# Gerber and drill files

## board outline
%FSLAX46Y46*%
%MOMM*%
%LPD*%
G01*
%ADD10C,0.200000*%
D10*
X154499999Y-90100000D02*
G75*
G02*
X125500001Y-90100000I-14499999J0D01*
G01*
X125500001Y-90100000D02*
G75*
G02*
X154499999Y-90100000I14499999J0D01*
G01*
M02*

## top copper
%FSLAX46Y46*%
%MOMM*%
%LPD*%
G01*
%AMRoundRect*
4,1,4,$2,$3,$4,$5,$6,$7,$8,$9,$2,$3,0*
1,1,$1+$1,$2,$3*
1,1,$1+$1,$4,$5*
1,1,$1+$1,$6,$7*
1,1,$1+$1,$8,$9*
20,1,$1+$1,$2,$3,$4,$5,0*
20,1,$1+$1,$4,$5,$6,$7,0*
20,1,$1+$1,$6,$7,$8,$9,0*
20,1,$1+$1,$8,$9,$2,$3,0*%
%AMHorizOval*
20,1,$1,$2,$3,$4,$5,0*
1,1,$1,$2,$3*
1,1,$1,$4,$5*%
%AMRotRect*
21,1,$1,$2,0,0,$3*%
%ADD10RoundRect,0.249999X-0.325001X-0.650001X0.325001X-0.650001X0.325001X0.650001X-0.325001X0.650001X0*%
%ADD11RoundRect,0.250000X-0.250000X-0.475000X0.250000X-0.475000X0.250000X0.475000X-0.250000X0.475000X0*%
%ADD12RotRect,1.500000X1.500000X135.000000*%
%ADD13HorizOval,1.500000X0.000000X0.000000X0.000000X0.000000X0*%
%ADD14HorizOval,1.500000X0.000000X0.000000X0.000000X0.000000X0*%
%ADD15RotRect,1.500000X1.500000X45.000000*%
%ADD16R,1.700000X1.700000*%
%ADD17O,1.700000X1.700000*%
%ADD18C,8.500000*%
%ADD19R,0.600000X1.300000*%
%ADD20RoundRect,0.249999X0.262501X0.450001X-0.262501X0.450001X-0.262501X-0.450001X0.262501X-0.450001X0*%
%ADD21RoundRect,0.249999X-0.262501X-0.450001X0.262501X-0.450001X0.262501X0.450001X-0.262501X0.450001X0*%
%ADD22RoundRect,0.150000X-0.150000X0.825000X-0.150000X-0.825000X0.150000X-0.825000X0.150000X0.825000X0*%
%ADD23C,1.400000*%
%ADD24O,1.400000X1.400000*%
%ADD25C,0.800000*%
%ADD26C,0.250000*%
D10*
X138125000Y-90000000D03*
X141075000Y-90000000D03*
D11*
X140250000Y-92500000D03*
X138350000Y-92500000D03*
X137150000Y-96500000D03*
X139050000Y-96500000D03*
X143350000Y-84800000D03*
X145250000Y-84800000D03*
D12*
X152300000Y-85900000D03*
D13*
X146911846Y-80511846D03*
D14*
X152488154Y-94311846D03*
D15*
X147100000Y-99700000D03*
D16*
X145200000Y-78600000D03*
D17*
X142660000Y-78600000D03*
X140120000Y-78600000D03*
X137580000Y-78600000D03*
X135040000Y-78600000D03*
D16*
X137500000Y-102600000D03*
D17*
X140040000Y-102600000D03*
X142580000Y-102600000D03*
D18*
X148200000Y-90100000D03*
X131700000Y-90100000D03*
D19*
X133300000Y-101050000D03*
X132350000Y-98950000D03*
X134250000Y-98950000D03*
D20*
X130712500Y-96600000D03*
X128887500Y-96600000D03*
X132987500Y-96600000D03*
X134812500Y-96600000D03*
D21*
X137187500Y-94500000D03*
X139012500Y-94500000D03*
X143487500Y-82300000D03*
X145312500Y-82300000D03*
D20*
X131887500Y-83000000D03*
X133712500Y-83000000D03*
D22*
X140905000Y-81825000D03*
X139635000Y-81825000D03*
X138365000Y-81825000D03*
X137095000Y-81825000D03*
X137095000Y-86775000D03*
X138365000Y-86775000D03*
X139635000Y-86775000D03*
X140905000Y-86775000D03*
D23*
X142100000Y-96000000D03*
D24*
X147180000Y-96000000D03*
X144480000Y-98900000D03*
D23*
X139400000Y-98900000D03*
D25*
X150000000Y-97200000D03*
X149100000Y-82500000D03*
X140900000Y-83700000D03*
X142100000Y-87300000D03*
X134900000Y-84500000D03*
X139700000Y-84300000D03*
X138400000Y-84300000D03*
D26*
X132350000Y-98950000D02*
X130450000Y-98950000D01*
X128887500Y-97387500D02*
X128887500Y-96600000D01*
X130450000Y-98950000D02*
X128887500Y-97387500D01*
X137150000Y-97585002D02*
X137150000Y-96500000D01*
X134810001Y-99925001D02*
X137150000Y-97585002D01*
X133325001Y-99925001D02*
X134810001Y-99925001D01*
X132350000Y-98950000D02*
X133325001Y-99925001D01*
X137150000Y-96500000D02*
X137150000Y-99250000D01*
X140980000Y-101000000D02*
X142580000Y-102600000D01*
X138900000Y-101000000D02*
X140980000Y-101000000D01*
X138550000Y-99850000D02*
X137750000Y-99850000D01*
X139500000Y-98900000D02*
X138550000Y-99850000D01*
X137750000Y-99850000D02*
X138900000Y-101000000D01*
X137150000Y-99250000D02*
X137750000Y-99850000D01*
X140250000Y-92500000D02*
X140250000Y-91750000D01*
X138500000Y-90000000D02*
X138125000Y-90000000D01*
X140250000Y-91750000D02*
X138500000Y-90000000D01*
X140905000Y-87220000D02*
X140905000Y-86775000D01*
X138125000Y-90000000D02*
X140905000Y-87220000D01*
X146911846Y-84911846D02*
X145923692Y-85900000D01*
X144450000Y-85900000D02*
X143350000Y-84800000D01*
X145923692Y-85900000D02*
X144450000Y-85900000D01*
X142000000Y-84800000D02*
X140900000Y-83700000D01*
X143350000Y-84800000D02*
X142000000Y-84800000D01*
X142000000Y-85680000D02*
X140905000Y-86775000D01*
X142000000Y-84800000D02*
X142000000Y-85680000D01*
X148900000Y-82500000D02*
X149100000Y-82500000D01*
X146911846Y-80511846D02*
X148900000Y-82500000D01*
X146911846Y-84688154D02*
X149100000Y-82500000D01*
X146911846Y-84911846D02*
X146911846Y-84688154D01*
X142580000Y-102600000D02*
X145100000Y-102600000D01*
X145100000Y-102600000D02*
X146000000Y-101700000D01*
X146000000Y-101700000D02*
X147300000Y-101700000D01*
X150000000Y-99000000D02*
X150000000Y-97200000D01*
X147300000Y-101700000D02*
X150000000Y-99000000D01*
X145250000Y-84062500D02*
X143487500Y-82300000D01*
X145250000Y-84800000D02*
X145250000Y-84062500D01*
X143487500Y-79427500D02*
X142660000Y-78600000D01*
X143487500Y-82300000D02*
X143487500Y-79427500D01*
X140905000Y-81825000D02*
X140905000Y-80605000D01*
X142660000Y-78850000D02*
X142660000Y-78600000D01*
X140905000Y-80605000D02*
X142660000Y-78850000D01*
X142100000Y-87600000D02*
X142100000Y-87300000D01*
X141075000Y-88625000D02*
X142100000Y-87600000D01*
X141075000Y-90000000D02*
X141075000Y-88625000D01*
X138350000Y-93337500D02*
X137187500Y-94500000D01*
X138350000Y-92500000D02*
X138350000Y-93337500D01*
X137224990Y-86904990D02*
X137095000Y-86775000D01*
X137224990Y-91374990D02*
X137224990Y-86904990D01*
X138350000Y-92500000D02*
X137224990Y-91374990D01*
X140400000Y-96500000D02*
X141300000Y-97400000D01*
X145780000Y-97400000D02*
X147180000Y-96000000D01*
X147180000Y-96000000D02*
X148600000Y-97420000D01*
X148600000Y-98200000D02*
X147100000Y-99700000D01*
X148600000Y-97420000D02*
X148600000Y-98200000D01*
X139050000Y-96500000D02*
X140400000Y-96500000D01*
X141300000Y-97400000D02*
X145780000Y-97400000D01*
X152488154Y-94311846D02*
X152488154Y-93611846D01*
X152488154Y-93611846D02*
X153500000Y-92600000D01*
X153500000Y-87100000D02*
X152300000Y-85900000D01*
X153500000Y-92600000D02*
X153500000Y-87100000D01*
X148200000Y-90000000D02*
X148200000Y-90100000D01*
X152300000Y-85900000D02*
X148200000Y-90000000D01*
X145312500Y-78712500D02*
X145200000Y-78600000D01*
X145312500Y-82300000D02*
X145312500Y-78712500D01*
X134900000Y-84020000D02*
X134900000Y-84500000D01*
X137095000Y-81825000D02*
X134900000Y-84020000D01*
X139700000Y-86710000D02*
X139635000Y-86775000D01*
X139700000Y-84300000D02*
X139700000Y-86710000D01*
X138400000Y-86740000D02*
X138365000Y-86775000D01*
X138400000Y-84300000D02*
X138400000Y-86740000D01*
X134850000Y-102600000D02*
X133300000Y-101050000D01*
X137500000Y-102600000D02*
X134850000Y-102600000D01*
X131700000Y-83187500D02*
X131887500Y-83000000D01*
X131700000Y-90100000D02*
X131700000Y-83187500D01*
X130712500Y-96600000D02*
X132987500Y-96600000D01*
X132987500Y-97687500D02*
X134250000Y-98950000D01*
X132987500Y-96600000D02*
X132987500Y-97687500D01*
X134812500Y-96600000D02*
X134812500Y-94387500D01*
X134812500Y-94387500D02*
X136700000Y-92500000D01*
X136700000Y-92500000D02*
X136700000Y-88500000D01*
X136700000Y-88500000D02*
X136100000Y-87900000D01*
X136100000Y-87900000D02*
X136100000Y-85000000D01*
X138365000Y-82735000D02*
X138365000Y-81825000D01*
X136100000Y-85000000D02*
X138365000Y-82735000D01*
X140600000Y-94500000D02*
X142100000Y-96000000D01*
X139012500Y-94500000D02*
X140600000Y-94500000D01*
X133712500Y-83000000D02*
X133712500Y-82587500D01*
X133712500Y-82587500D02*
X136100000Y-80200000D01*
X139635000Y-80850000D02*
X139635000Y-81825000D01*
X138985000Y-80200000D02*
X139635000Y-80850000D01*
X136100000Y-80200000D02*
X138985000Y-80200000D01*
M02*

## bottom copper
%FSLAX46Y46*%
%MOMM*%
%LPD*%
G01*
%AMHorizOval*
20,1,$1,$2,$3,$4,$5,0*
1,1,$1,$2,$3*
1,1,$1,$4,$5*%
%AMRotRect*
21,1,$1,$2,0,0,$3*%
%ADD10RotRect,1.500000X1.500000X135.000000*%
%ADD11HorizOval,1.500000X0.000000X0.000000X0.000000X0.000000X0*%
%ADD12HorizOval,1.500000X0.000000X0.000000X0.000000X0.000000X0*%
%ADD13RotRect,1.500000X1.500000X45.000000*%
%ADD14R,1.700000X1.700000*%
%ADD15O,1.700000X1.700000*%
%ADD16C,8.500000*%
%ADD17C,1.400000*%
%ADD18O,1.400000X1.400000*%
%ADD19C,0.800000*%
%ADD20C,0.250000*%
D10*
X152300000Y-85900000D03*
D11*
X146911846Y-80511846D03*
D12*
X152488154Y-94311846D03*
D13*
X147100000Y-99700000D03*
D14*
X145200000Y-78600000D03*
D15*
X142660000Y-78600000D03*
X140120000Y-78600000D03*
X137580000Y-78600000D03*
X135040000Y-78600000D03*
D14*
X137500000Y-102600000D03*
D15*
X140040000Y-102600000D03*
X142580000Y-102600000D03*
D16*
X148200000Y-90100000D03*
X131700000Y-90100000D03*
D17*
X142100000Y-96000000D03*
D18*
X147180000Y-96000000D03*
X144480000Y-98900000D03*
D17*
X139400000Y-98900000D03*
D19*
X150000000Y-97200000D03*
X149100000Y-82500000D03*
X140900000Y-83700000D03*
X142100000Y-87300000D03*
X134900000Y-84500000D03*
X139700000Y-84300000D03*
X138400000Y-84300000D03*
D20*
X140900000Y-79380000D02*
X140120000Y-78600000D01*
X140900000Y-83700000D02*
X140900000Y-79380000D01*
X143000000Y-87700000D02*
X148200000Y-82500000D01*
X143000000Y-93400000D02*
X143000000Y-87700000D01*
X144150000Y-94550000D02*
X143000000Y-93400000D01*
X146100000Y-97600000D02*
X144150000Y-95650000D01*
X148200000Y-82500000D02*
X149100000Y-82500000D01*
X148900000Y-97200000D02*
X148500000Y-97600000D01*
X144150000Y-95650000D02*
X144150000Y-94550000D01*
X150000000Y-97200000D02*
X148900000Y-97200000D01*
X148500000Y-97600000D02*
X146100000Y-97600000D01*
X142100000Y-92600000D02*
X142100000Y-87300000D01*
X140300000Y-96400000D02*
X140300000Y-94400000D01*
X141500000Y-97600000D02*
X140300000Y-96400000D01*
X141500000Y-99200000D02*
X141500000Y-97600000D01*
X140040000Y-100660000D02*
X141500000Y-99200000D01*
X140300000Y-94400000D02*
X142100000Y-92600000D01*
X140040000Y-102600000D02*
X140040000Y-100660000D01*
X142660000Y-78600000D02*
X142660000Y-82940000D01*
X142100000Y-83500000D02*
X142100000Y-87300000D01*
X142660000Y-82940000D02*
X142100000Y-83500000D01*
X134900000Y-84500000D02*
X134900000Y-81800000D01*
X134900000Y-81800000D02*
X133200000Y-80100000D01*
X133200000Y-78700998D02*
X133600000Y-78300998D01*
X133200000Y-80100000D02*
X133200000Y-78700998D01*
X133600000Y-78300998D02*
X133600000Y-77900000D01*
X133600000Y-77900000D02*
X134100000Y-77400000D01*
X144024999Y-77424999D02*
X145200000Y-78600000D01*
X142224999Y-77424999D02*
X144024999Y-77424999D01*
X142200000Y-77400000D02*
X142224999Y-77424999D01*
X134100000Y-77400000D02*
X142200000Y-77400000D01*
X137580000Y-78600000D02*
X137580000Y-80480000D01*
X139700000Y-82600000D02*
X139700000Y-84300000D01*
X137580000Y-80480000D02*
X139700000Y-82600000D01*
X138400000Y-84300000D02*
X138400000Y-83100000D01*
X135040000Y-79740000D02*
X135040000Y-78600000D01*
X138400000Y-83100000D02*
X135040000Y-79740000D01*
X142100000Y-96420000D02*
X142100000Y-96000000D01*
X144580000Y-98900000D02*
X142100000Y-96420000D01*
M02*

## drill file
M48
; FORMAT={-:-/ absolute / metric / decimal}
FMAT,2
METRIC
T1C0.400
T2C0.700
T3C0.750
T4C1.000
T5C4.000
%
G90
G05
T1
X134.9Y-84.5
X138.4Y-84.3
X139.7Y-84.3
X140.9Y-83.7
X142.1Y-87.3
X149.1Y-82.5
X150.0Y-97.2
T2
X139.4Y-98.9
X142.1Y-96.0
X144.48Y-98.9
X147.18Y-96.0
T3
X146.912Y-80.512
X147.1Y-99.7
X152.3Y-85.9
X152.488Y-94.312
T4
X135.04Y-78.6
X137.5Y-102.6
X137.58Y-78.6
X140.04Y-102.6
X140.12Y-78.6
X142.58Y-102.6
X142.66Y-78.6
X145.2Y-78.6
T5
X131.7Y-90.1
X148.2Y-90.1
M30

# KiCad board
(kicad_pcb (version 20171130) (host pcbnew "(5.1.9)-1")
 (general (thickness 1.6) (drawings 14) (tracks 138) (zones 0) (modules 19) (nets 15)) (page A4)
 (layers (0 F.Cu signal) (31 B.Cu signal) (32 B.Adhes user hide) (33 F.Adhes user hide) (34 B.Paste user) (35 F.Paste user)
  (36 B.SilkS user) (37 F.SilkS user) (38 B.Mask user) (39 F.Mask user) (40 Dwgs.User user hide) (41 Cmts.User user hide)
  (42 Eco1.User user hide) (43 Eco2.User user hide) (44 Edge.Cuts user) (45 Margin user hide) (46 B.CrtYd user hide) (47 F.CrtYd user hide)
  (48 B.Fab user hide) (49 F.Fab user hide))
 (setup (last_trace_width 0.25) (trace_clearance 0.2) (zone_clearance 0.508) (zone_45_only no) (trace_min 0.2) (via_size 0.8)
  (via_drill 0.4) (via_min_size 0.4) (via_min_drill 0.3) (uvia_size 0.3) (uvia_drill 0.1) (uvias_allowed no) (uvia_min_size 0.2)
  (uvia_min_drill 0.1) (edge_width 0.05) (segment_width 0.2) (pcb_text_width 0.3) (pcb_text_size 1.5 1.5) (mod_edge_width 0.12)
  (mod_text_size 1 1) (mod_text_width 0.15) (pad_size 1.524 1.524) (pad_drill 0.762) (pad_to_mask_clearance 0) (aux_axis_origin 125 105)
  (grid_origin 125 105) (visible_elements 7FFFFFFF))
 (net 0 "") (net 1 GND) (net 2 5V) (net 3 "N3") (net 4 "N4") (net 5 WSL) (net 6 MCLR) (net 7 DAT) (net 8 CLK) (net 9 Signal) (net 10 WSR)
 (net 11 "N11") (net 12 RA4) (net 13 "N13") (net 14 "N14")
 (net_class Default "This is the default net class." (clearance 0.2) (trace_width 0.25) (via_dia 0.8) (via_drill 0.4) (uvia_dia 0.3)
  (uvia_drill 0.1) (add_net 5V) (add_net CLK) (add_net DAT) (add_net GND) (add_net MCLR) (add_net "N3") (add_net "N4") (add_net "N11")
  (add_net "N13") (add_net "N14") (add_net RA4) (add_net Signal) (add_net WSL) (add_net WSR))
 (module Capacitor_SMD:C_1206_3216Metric (layer F.Cu) (at 139.6 90)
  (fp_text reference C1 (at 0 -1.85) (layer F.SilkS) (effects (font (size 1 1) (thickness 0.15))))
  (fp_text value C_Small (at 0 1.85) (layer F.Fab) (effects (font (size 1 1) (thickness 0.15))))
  (pad 1 smd roundrect (at -1.475 0) (size 1.15 1.8) (layers F.Cu F.Paste F.Mask) (roundrect_rratio 0.2173904347826087) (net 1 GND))
  (pad 2 smd roundrect (at 1.475 0) (size 1.15 1.8) (layers F.Cu F.Paste F.Mask) (roundrect_rratio 0.2173904347826087) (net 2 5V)))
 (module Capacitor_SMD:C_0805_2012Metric (layer F.Cu) (at 139.3 92.5)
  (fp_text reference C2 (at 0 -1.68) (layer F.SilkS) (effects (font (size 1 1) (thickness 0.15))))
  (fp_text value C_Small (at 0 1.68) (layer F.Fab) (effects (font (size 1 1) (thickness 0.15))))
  (pad 2 smd roundrect (at 0.95 0) (size 1 1.45) (layers F.Cu F.Paste F.Mask) (roundrect_rratio 0.25) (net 1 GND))
  (pad 1 smd roundrect (at -0.95 0) (size 1 1.45) (layers F.Cu F.Paste F.Mask) (roundrect_rratio 0.25) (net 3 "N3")))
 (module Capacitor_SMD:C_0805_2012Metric (layer F.Cu) (at 138.1 96.5)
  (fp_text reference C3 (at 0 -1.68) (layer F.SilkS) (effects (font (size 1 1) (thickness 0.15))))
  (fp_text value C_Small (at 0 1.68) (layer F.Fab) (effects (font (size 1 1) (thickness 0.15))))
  (pad 1 smd roundrect (at -0.95 0) (size 1 1.45) (layers F.Cu F.Paste F.Mask) (roundrect_rratio 0.25) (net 1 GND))
  (pad 2 smd roundrect (at 0.95 0) (size 1 1.45) (layers F.Cu F.Paste F.Mask) (roundrect_rratio 0.25) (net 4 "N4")))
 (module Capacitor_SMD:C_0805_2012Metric (layer F.Cu) (at 144.3 84.8)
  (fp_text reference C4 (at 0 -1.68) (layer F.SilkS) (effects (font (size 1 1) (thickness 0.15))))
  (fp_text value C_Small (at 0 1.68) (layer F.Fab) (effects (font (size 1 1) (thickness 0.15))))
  (pad 1 smd roundrect (at -0.95 0) (size 1 1.45) (layers F.Cu F.Paste F.Mask) (roundrect_rratio 0.25) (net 1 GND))
  (pad 2 smd roundrect (at 0.95 0) (size 1 1.45) (layers F.Cu F.Paste F.Mask) (roundrect_rratio 0.25) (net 2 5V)))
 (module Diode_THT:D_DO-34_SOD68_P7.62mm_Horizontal (layer F.Cu) (at 152.3 85.9 135)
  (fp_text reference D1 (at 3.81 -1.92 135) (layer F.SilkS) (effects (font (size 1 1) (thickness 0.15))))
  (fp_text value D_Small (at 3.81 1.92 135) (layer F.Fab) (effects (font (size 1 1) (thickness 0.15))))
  (pad 1 thru_hole rect (at 0 0 135) (size 1.5 1.5) (drill 0.75) (layers *.Cu *.Mask) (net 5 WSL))
  (pad 2 thru_hole oval (at 7.62 0 135) (size 1.5 1.5) (drill 0.75) (layers *.Cu *.Mask) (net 1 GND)))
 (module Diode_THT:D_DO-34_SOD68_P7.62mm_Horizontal (layer F.Cu) (at 147.1 99.7 45)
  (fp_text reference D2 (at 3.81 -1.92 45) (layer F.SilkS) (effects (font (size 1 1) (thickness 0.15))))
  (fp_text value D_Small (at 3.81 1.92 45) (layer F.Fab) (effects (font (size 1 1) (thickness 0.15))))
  (pad 2 thru_hole oval (at 7.62 0 45) (size 1.5 1.5) (drill 0.75) (layers *.Cu *.Mask) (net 5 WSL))
  (pad 1 thru_hole rect (at 0 0 45) (size 1.5 1.5) (drill 0.75) (layers *.Cu *.Mask) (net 4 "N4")))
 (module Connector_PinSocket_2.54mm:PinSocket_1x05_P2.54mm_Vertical (layer F.Cu) (at 145.2 78.6 270)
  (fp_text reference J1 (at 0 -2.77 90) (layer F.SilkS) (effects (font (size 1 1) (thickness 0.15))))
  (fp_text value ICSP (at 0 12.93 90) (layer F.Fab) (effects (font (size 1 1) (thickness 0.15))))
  (pad 1 thru_hole rect (at 0 0 270) (size 1.7 1.7) (drill 1) (layers *.Cu *.Mask) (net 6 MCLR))
  (pad 2 thru_hole oval (at 0 2.54 270) (size 1.7 1.7) (drill 1) (layers *.Cu *.Mask) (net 2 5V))
  (pad 3 thru_hole oval (at 0 5.08 270) (size 1.7 1.7) (drill 1) (layers *.Cu *.Mask) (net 1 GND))
  (pad 4 thru_hole oval (at 0 7.62 270) (size 1.7 1.7) (drill 1) (layers *.Cu *.Mask) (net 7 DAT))
  (pad 5 thru_hole oval (at 0 10.16 270) (size 1.7 1.7) (drill 1) (layers *.Cu *.Mask) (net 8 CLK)))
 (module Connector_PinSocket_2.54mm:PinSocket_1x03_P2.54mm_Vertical (layer F.Cu) (at 137.5 102.6 90)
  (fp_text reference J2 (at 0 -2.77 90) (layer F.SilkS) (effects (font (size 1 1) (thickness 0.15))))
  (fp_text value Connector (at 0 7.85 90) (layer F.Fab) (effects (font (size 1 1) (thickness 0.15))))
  (pad 1 thru_hole rect (at 0 0 90) (size 1.7 1.7) (drill 1) (layers *.Cu *.Mask) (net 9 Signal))
  (pad 2 thru_hole oval (at 0 2.54 90) (size 1.7 1.7) (drill 1) (layers *.Cu *.Mask) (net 2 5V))
  (pad 3 thru_hole oval (at 0 5.08 90) (size 1.7 1.7) (drill 1) (layers *.Cu *.Mask) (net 1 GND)))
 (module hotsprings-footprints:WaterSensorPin (layer F.Cu) (at 148.2 90.1)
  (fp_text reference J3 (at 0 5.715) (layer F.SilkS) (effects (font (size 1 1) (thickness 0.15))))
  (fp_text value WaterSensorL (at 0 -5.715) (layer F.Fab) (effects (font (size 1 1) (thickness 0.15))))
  (pad 1 thru_hole circle (at 0 0) (size 8.5 8.5) (drill 4) (layers *.Cu *.Mask) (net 5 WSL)))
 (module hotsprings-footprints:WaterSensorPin (layer F.Cu) (at 131.7 90.1)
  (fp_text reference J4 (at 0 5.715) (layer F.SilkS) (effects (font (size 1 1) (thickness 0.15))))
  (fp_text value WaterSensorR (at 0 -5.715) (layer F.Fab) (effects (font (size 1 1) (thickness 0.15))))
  (pad 1 thru_hole circle (at 0 0) (size 8.5 8.5) (drill 4) (layers *.Cu *.Mask) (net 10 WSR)))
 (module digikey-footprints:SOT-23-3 (layer F.Cu) (at 133.3 100 270)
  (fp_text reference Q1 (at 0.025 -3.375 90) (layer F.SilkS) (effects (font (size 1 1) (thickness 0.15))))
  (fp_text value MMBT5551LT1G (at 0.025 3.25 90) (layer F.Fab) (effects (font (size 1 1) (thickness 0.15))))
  (pad 3 smd rect (at 1.05 0 270) (size 1.3 0.6) (layers F.Cu F.Paste F.Mask) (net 9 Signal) (solder_mask_margin 0.07))
  (pad 2 smd rect (at -1.05 0.95 270) (size 1.3 0.6) (layers F.Cu F.Paste F.Mask) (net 1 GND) (solder_mask_margin 0.07))
  (pad 1 smd rect (at -1.05 -0.95 270) (size 1.3 0.6) (layers F.Cu F.Paste F.Mask) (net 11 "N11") (solder_mask_margin 0.07)))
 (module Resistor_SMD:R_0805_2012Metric (layer F.Cu) (at 129.8 96.6 180)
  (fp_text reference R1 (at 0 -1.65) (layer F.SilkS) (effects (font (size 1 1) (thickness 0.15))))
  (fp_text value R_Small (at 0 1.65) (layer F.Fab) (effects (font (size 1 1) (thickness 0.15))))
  (pad 1 smd roundrect (at -0.9125 0 180) (size 1.025 1.4) (layers F.Cu F.Paste F.Mask) (roundrect_rratio 0.2439014634146341) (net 11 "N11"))
  (pad 2 smd roundrect (at 0.9125 0 180) (size 1.025 1.4) (layers F.Cu F.Paste F.Mask) (roundrect_rratio 0.2439014634146341) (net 1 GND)))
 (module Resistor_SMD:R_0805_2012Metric (layer F.Cu) (at 133.9 96.6 180)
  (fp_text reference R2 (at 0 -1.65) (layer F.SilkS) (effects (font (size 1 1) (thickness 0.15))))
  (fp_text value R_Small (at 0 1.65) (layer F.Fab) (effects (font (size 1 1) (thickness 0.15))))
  (pad 2 smd roundrect (at 0.9125 0 180) (size 1.025 1.4) (layers F.Cu F.Paste F.Mask) (roundrect_rratio 0.2439014634146341) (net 11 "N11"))
  (pad 1 smd roundrect (at -0.9125 0 180) (size 1.025 1.4) (layers F.Cu F.Paste F.Mask) (roundrect_rratio 0.2439014634146341) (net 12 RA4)))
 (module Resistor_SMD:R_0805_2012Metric (layer F.Cu) (at 138.1 94.5)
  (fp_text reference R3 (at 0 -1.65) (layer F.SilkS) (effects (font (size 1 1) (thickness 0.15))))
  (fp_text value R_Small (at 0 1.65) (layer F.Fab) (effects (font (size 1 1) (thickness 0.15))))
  (pad 1 smd roundrect (at -0.9125 0) (size 1.025 1.4) (layers F.Cu F.Paste F.Mask) (roundrect_rratio 0.2439014634146341) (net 3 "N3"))
  (pad 2 smd roundrect (at 0.9125 0) (size 1.025 1.4) (layers F.Cu F.Paste F.Mask) (roundrect_rratio 0.2439014634146341) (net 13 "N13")))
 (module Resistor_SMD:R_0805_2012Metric (layer F.Cu) (at 144.4 82.3)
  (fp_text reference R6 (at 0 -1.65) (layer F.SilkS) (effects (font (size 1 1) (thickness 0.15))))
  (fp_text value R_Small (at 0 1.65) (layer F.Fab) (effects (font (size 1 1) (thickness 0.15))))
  (pad 1 smd roundrect (at -0.9125 0) (size 1.025 1.4) (layers F.Cu F.Paste F.Mask) (roundrect_rratio 0.2439014634146341) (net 2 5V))
  (pad 2 smd roundrect (at 0.9125 0) (size 1.025 1.4) (layers F.Cu F.Paste F.Mask) (roundrect_rratio 0.2439014634146341) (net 6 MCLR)))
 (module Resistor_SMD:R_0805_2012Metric (layer F.Cu) (at 132.8 83 180)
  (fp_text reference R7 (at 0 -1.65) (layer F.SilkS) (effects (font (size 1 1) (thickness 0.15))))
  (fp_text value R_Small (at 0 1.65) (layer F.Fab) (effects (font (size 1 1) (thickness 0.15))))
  (pad 2 smd roundrect (at 0.9125 0 180) (size 1.025 1.4) (layers F.Cu F.Paste F.Mask) (roundrect_rratio 0.2439014634146341) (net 10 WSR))
  (pad 1 smd roundrect (at -0.9125 0 180) (size 1.025 1.4) (layers F.Cu F.Paste F.Mask) (roundrect_rratio 0.2439014634146341) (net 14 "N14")))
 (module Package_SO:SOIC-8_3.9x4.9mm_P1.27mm (layer F.Cu) (at 139 84.3 270)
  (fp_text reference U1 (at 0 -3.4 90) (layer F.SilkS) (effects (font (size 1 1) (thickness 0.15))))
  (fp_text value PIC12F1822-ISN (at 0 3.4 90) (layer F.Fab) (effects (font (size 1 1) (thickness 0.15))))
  (pad 1 smd roundrect (at -2.475 -1.905 270) (size 1.95 0.6) (layers F.Cu F.Paste F.Mask) (roundrect_rratio 0.25) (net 2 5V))
  (pad 2 smd roundrect (at -2.475 -0.635 270) (size 1.95 0.6) (layers F.Cu F.Paste F.Mask) (roundrect_rratio 0.25) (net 14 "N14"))
  (pad 3 smd roundrect (at -2.475 0.635 270) (size 1.95 0.6) (layers F.Cu F.Paste F.Mask) (roundrect_rratio 0.25) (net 12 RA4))
  (pad 4 smd roundrect (at -2.475 1.905 270) (size 1.95 0.6) (layers F.Cu F.Paste F.Mask) (roundrect_rratio 0.25) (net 6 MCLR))
  (pad 5 smd roundrect (at 2.475 1.905 270) (size 1.95 0.6) (layers F.Cu F.Paste F.Mask) (roundrect_rratio 0.25) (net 3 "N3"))
  (pad 6 smd roundrect (at 2.475 0.635 270) (size 1.95 0.6) (layers F.Cu F.Paste F.Mask) (roundrect_rratio 0.25) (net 8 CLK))
  (pad 7 smd roundrect (at 2.475 -0.635 270) (size 1.95 0.6) (layers F.Cu F.Paste F.Mask) (roundrect_rratio 0.25) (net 7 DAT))
  (pad 8 smd roundrect (at 2.475 -1.905 270) (size 1.95 0.6) (layers F.Cu F.Paste F.Mask) (roundrect_rratio 0.25) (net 1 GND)))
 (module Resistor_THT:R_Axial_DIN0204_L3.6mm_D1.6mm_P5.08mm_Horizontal (layer F.Cu) (at 142.1 96)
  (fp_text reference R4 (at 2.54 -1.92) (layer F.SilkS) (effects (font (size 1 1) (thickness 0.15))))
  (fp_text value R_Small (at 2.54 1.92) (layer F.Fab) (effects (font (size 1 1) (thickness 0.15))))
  (pad 1 thru_hole circle (at 0 0) (size 1.4 1.4) (drill 0.7) (layers *.Cu *.Mask) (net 13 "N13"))
  (pad 2 thru_hole oval (at 5.08 0) (size 1.4 1.4) (drill 0.7) (layers *.Cu *.Mask) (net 4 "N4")))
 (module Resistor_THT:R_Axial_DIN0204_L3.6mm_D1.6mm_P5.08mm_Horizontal (layer F.Cu) (at 139.4 98.9)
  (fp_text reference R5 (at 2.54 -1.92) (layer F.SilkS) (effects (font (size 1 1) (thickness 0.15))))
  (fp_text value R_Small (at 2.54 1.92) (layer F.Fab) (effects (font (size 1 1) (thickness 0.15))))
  (pad 2 thru_hole oval (at 5.08 0) (size 1.4 1.4) (drill 0.7) (layers *.Cu *.Mask) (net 13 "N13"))
  (pad 1 thru_hole circle (at 0 0) (size 1.4 1.4) (drill 0.7) (layers *.Cu *.Mask) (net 1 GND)))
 (gr_circle (center 140 90.1) (end 154.499999 90.1) (layer Edge.Cuts) (width 0.2))
 (via (at 150 97.2) (size 0.8) (drill 0.4) (layers F.Cu B.Cu) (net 1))
 (via (at 149.1 82.5) (size 0.8) (drill 0.4) (layers F.Cu B.Cu) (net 1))
 (via (at 140.9 83.7) (size 0.8) (drill 0.4) (layers F.Cu B.Cu) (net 1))
 (segment (start 132.35 98.95) (end 130.45 98.95) (width 0.25) (layer F.Cu) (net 1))
 (segment (start 128.8875 97.3875) (end 128.8875 96.6) (width 0.25) (layer F.Cu) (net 1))
 (segment (start 130.45 98.95) (end 128.8875 97.3875) (width 0.25) (layer F.Cu) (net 1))
 (segment (start 137.15 97.585002) (end 137.15 96.5) (width 0.25) (layer F.Cu) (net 1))
 (segment (start 134.810001 99.925001) (end 137.15 97.585002) (width 0.25) (layer F.Cu) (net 1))
 (segment (start 133.325001 99.925001) (end 134.810001 99.925001) (width 0.25) (layer F.Cu) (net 1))
 (segment (start 132.35 98.95) (end 133.325001 99.925001) (width 0.25) (layer F.Cu) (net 1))
 (segment (start 137.15 96.5) (end 137.15 99.25) (width 0.25) (layer F.Cu) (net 1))
 (segment (start 140.98 101) (end 142.58 102.6) (width 0.25) (layer F.Cu) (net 1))
 (segment (start 138.9 101) (end 140.98 101) (width 0.25) (layer F.Cu) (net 1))
 (segment (start 138.55 99.85) (end 137.75 99.85) (width 0.25) (layer F.Cu) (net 1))
 (segment (start 139.5 98.9) (end 138.55 99.85) (width 0.25) (layer F.Cu) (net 1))
 (segment (start 137.75 99.85) (end 138.9 101) (width 0.25) (layer F.Cu) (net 1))
 (segment (start 137.15 99.25) (end 137.75 99.85) (width 0.25) (layer F.Cu) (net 1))
 (segment (start 140.25 92.5) (end 140.25 91.75) (width 0.25) (layer F.Cu) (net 1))
 (segment (start 138.5 90) (end 138.125 90) (width 0.25) (layer F.Cu) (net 1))
 (segment (start 140.25 91.75) (end 138.5 90) (width 0.25) (layer F.Cu) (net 1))
 (segment (start 140.905 87.22) (end 140.905 86.775) (width 0.25) (layer F.Cu) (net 1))
 (segment (start 138.125 90) (end 140.905 87.22) (width 0.25) (layer F.Cu) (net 1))
 (segment (start 146.911846 84.911846) (end 145.923692 85.9) (width 0.25) (layer F.Cu) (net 1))
 (segment (start 144.45 85.9) (end 143.35 84.8) (width 0.25) (layer F.Cu) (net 1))
 (segment (start 145.923692 85.9) (end 144.45 85.9) (width 0.25) (layer F.Cu) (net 1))
 (segment (start 142 84.8) (end 140.9 83.7) (width 0.25) (layer F.Cu) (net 1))
 (segment (start 143.35 84.8) (end 142 84.8) (width 0.25) (layer F.Cu) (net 1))
 (segment (start 142 85.68) (end 140.905 86.775) (width 0.25) (layer F.Cu) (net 1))
 (segment (start 142 84.8) (end 142 85.68) (width 0.25) (layer F.Cu) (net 1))
 (segment (start 140.9 79.38) (end 140.12 78.6) (width 0.25) (layer B.Cu) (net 1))
 (segment (start 140.9 83.7) (end 140.9 79.38) (width 0.25) (layer B.Cu) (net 1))
 (segment (start 148.9 82.5) (end 149.1 82.5) (width 0.25) (layer F.Cu) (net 1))
 (segment (start 146.911846 80.511846) (end 148.9 82.5) (width 0.25) (layer F.Cu) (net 1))
 (segment (start 146.911846 84.688154) (end 149.1 82.5) (width 0.25) (layer F.Cu) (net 1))
 (segment (start 146.911846 84.911846) (end 146.911846 84.688154) (width 0.25) (layer F.Cu) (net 1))
 (segment (start 142.58 102.6) (end 145.1 102.6) (width 0.25) (layer F.Cu) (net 1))
 (segment (start 145.1 102.6) (end 146 101.7) (width 0.25) (layer F.Cu) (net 1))
 (segment (start 146 101.7) (end 147.3 101.7) (width 0.25) (layer F.Cu) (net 1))
 (segment (start 150 99) (end 150 97.2) (width 0.25) (layer F.Cu) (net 1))
 (segment (start 147.3 101.7) (end 150 99) (width 0.25) (layer F.Cu) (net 1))
 (segment (start 143 87.7) (end 148.2 82.5) (width 0.25) (layer B.Cu) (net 1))
 (segment (start 143 93.4) (end 143 87.7) (width 0.25) (layer B.Cu) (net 1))
 (segment (start 144.15 94.55) (end 143 93.4) (width 0.25) (layer B.Cu) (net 1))
 (segment (start 146.1 97.6) (end 144.15 95.65) (width 0.25) (layer B.Cu) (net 1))
 (segment (start 148.2 82.5) (end 149.1 82.5) (width 0.25) (layer B.Cu) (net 1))
 (segment (start 148.9 97.2) (end 148.5 97.6) (width 0.25) (layer B.Cu) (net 1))
 (segment (start 144.15 95.65) (end 144.15 94.55) (width 0.25) (layer B.Cu) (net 1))
 (segment (start 150 97.2) (end 148.9 97.2) (width 0.25) (layer B.Cu) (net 1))
 (segment (start 148.5 97.6) (end 146.1 97.6) (width 0.25) (layer B.Cu) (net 1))
 (via (at 142.1 87.3) (size 0.8) (drill 0.4) (layers F.Cu B.Cu) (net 2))
 (segment (start 145.25 84.0625) (end 143.4875 82.3) (width 0.25) (layer F.Cu) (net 2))
 (segment (start 145.25 84.8) (end 145.25 84.0625) (width 0.25) (layer F.Cu) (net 2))
 (segment (start 143.4875 79.4275) (end 142.66 78.6) (width 0.25) (layer F.Cu) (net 2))
 (segment (start 143.4875 82.3) (end 143.4875 79.4275) (width 0.25) (layer F.Cu) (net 2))
 (segment (start 140.905 81.825) (end 140.905 80.605) (width 0.25) (layer F.Cu) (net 2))
 (segment (start 142.66 78.85) (end 142.66 78.6) (width 0.25) (layer F.Cu) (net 2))
 (segment (start 140.905 80.605) (end 142.66 78.85) (width 0.25) (layer F.Cu) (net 2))
 (segment (start 142.1 87.6) (end 142.1 87.3) (width 0.25) (layer F.Cu) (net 2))
 (segment (start 141.075 88.625) (end 142.1 87.6) (width 0.25) (layer F.Cu) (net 2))
 (segment (start 141.075 90) (end 141.075 88.625) (width 0.25) (layer F.Cu) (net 2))
 (segment (start 142.1 92.6) (end 142.1 87.3) (width 0.25) (layer B.Cu) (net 2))
 (segment (start 140.3 96.4) (end 140.3 94.4) (width 0.25) (layer B.Cu) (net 2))
 (segment (start 141.5 97.6) (end 140.3 96.4) (width 0.25) (layer B.Cu) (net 2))
 (segment (start 141.5 99.2) (end 141.5 97.6) (width 0.25) (layer B.Cu) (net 2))
 (segment (start 140.04 100.66) (end 141.5 99.2) (width 0.25) (layer B.Cu) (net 2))
 (segment (start 140.3 94.4) (end 142.1 92.6) (width 0.25) (layer B.Cu) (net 2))
 (segment (start 140.04 102.6) (end 140.04 100.66) (width 0.25) (layer B.Cu) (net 2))
 (segment (start 142.66 78.6) (end 142.66 82.94) (width 0.25) (layer B.Cu) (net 2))
 (segment (start 142.1 83.5) (end 142.1 87.3) (width 0.25) (layer B.Cu) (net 2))
 (segment (start 142.66 82.94) (end 142.1 83.5) (width 0.25) (layer B.Cu) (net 2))
 (segment (start 138.35 93.3375) (end 137.1875 94.5) (width 0.25) (layer F.Cu) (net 3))
 (segment (start 138.35 92.5) (end 138.35 93.3375) (width 0.25) (layer F.Cu) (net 3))
 (segment (start 137.22499 86.90499) (end 137.095 86.775) (width 0.25) (layer F.Cu) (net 3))
 (segment (start 137.22499 91.37499) (end 137.22499 86.90499) (width 0.25) (layer F.Cu) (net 3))
 (segment (start 138.35 92.5) (end 137.22499 91.37499) (width 0.25) (layer F.Cu) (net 3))
 (segment (start 140.4 96.5) (end 141.3 97.4) (width 0.25) (layer F.Cu) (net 4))
 (segment (start 145.78 97.4) (end 147.18 96) (width 0.25) (layer F.Cu) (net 4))
 (segment (start 147.18 96) (end 148.6 97.42) (width 0.25) (layer F.Cu) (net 4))
 (segment (start 148.6 98.2) (end 147.1 99.7) (width 0.25) (layer F.Cu) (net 4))
 (segment (start 148.6 97.42) (end 148.6 98.2) (width 0.25) (layer F.Cu) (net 4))
 (segment (start 139.05 96.5) (end 140.4 96.5) (width 0.25) (layer F.Cu) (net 4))
 (segment (start 141.3 97.4) (end 145.78 97.4) (width 0.25) (layer F.Cu) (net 4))
 (segment (start 152.488154 94.311846) (end 152.488154 93.611846) (width 0.25) (layer F.Cu) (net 5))
 (segment (start 152.488154 93.611846) (end 153.5 92.6) (width 0.25) (layer F.Cu) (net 5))
 (segment (start 153.5 87.1) (end 152.3 85.9) (width 0.25) (layer F.Cu) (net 5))
 (segment (start 153.5 92.6) (end 153.5 87.1) (width 0.25) (layer F.Cu) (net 5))
 (segment (start 148.2 90) (end 148.2 90.1) (width 0.25) (layer F.Cu) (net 5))
 (segment (start 152.3 85.9) (end 148.2 90) (width 0.25) (layer F.Cu) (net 5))
 (via (at 134.9 84.5) (size 0.8) (drill 0.4) (layers F.Cu B.Cu) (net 6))
 (segment (start 145.3125 78.7125) (end 145.2 78.6) (width 0.25) (layer F.Cu) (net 6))
 (segment (start 145.3125 82.3) (end 145.3125 78.7125) (width 0.25) (layer F.Cu) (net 6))
 (segment (start 134.9 84.02) (end 134.9 84.5) (width 0.25) (layer F.Cu) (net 6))
 (segment (start 137.095 81.825) (end 134.9 84.02) (width 0.25) (layer F.Cu) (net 6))
 (segment (start 134.9 84.5) (end 134.9 81.8) (width 0.25) (layer B.Cu) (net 6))
 (segment (start 134.9 81.8) (end 133.2 80.1) (width 0.25) (layer B.Cu) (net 6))
 (segment (start 133.2 78.700998) (end 133.6 78.300998) (width 0.25) (layer B.Cu) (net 6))
 (segment (start 133.2 80.1) (end 133.2 78.700998) (width 0.25) (layer B.Cu) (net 6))
 (segment (start 133.6 78.300998) (end 133.6 77.9) (width 0.25) (layer B.Cu) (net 6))
 (segment (start 133.6 77.9) (end 134.1 77.4) (width 0.25) (layer B.Cu) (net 6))
 (segment (start 144.024999 77.424999) (end 145.2 78.6) (width 0.25) (layer B.Cu) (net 6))
 (segment (start 142.224999 77.424999) (end 144.024999 77.424999) (width 0.25) (layer B.Cu) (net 6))
 (segment (start 142.2 77.4) (end 142.224999 77.424999) (width 0.25) (layer B.Cu) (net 6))
 (segment (start 134.1 77.4) (end 142.2 77.4) (width 0.25) (layer B.Cu) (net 6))
 (via (at 139.7 84.3) (size 0.8) (drill 0.4) (layers F.Cu B.Cu) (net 7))
 (segment (start 137.58 78.6) (end 137.58 80.48) (width 0.25) (layer B.Cu) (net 7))
 (segment (start 139.7 82.6) (end 139.7 84.3) (width 0.25) (layer B.Cu) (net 7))
 (segment (start 137.58 80.48) (end 139.7 82.6) (width 0.25) (layer B.Cu) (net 7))
 (segment (start 139.7 86.71) (end 139.635 86.775) (width 0.25) (layer F.Cu) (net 7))
 (segment (start 139.7 84.3) (end 139.7 86.71) (width 0.25) (layer F.Cu) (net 7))
 (via (at 138.4 84.3) (size 0.8) (drill 0.4) (layers F.Cu B.Cu) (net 8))
 (segment (start 138.4 84.3) (end 138.4 83.1) (width 0.25) (layer B.Cu) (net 8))
 (segment (start 135.04 79.74) (end 135.04 78.6) (width 0.25) (layer B.Cu) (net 8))
 (segment (start 138.4 83.1) (end 135.04 79.74) (width 0.25) (layer B.Cu) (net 8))
 (segment (start 138.4 86.74) (end 138.365 86.775) (width 0.25) (layer F.Cu) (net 8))
 (segment (start 138.4 84.3) (end 138.4 86.74) (width 0.25) (layer F.Cu) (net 8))
 (segment (start 134.85 102.6) (end 133.3 101.05) (width 0.25) (layer F.Cu) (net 9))
 (segment (start 137.5 102.6) (end 134.85 102.6) (width 0.25) (layer F.Cu) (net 9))
 (segment (start 131.7 83.1875) (end 131.8875 83) (width 0.25) (layer F.Cu) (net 10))
 (segment (start 131.7 90.1) (end 131.7 83.1875) (width 0.25) (layer F.Cu) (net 10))
 (segment (start 130.7125 96.6) (end 132.9875 96.6) (width 0.25) (layer F.Cu) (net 11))
 (segment (start 132.9875 97.6875) (end 134.25 98.95) (width 0.25) (layer F.Cu) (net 11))
 (segment (start 132.9875 96.6) (end 132.9875 97.6875) (width 0.25) (layer F.Cu) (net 11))
 (segment (start 134.8125 96.6) (end 134.8125 94.3875) (width 0.25) (layer F.Cu) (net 12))
 (segment (start 134.8125 94.3875) (end 136.7 92.5) (width 0.25) (layer F.Cu) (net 12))
 (segment (start 136.7 92.5) (end 136.7 88.5) (width 0.25) (layer F.Cu) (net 12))
 (segment (start 136.7 88.5) (end 136.1 87.9) (width 0.25) (layer F.Cu) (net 12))
 (segment (start 136.1 87.9) (end 136.1 85) (width 0.25) (layer F.Cu) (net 12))
 (segment (start 138.365 82.735) (end 138.365 81.825) (width 0.25) (layer F.Cu) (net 12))
 (segment (start 136.1 85) (end 138.365 82.735) (width 0.25) (layer F.Cu) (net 12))
 (segment (start 140.6 94.5) (end 142.1 96) (width 0.25) (layer F.Cu) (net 13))
 (segment (start 139.0125 94.5) (end 140.6 94.5) (width 0.25) (layer F.Cu) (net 13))
 (segment (start 142.1 96.42) (end 142.1 96) (width 0.25) (layer B.Cu) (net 13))
 (segment (start 144.58 98.9) (end 142.1 96.42) (width 0.25) (layer B.Cu) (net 13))
 (segment (start 133.7125 83) (end 133.7125 82.5875) (width 0.25) (layer F.Cu) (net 14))
 (segment (start 133.7125 82.5875) (end 136.1 80.2) (width 0.25) (layer F.Cu) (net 14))
 (segment (start 139.635 80.85) (end 139.635 81.825) (width 0.25) (layer F.Cu) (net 14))
 (segment (start 138.985 80.2) (end 139.635 80.85) (width 0.25) (layer F.Cu) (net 14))
 (segment (start 136.1 80.2) (end 138.985 80.2) (width 0.25) (layer F.Cu) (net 14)))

